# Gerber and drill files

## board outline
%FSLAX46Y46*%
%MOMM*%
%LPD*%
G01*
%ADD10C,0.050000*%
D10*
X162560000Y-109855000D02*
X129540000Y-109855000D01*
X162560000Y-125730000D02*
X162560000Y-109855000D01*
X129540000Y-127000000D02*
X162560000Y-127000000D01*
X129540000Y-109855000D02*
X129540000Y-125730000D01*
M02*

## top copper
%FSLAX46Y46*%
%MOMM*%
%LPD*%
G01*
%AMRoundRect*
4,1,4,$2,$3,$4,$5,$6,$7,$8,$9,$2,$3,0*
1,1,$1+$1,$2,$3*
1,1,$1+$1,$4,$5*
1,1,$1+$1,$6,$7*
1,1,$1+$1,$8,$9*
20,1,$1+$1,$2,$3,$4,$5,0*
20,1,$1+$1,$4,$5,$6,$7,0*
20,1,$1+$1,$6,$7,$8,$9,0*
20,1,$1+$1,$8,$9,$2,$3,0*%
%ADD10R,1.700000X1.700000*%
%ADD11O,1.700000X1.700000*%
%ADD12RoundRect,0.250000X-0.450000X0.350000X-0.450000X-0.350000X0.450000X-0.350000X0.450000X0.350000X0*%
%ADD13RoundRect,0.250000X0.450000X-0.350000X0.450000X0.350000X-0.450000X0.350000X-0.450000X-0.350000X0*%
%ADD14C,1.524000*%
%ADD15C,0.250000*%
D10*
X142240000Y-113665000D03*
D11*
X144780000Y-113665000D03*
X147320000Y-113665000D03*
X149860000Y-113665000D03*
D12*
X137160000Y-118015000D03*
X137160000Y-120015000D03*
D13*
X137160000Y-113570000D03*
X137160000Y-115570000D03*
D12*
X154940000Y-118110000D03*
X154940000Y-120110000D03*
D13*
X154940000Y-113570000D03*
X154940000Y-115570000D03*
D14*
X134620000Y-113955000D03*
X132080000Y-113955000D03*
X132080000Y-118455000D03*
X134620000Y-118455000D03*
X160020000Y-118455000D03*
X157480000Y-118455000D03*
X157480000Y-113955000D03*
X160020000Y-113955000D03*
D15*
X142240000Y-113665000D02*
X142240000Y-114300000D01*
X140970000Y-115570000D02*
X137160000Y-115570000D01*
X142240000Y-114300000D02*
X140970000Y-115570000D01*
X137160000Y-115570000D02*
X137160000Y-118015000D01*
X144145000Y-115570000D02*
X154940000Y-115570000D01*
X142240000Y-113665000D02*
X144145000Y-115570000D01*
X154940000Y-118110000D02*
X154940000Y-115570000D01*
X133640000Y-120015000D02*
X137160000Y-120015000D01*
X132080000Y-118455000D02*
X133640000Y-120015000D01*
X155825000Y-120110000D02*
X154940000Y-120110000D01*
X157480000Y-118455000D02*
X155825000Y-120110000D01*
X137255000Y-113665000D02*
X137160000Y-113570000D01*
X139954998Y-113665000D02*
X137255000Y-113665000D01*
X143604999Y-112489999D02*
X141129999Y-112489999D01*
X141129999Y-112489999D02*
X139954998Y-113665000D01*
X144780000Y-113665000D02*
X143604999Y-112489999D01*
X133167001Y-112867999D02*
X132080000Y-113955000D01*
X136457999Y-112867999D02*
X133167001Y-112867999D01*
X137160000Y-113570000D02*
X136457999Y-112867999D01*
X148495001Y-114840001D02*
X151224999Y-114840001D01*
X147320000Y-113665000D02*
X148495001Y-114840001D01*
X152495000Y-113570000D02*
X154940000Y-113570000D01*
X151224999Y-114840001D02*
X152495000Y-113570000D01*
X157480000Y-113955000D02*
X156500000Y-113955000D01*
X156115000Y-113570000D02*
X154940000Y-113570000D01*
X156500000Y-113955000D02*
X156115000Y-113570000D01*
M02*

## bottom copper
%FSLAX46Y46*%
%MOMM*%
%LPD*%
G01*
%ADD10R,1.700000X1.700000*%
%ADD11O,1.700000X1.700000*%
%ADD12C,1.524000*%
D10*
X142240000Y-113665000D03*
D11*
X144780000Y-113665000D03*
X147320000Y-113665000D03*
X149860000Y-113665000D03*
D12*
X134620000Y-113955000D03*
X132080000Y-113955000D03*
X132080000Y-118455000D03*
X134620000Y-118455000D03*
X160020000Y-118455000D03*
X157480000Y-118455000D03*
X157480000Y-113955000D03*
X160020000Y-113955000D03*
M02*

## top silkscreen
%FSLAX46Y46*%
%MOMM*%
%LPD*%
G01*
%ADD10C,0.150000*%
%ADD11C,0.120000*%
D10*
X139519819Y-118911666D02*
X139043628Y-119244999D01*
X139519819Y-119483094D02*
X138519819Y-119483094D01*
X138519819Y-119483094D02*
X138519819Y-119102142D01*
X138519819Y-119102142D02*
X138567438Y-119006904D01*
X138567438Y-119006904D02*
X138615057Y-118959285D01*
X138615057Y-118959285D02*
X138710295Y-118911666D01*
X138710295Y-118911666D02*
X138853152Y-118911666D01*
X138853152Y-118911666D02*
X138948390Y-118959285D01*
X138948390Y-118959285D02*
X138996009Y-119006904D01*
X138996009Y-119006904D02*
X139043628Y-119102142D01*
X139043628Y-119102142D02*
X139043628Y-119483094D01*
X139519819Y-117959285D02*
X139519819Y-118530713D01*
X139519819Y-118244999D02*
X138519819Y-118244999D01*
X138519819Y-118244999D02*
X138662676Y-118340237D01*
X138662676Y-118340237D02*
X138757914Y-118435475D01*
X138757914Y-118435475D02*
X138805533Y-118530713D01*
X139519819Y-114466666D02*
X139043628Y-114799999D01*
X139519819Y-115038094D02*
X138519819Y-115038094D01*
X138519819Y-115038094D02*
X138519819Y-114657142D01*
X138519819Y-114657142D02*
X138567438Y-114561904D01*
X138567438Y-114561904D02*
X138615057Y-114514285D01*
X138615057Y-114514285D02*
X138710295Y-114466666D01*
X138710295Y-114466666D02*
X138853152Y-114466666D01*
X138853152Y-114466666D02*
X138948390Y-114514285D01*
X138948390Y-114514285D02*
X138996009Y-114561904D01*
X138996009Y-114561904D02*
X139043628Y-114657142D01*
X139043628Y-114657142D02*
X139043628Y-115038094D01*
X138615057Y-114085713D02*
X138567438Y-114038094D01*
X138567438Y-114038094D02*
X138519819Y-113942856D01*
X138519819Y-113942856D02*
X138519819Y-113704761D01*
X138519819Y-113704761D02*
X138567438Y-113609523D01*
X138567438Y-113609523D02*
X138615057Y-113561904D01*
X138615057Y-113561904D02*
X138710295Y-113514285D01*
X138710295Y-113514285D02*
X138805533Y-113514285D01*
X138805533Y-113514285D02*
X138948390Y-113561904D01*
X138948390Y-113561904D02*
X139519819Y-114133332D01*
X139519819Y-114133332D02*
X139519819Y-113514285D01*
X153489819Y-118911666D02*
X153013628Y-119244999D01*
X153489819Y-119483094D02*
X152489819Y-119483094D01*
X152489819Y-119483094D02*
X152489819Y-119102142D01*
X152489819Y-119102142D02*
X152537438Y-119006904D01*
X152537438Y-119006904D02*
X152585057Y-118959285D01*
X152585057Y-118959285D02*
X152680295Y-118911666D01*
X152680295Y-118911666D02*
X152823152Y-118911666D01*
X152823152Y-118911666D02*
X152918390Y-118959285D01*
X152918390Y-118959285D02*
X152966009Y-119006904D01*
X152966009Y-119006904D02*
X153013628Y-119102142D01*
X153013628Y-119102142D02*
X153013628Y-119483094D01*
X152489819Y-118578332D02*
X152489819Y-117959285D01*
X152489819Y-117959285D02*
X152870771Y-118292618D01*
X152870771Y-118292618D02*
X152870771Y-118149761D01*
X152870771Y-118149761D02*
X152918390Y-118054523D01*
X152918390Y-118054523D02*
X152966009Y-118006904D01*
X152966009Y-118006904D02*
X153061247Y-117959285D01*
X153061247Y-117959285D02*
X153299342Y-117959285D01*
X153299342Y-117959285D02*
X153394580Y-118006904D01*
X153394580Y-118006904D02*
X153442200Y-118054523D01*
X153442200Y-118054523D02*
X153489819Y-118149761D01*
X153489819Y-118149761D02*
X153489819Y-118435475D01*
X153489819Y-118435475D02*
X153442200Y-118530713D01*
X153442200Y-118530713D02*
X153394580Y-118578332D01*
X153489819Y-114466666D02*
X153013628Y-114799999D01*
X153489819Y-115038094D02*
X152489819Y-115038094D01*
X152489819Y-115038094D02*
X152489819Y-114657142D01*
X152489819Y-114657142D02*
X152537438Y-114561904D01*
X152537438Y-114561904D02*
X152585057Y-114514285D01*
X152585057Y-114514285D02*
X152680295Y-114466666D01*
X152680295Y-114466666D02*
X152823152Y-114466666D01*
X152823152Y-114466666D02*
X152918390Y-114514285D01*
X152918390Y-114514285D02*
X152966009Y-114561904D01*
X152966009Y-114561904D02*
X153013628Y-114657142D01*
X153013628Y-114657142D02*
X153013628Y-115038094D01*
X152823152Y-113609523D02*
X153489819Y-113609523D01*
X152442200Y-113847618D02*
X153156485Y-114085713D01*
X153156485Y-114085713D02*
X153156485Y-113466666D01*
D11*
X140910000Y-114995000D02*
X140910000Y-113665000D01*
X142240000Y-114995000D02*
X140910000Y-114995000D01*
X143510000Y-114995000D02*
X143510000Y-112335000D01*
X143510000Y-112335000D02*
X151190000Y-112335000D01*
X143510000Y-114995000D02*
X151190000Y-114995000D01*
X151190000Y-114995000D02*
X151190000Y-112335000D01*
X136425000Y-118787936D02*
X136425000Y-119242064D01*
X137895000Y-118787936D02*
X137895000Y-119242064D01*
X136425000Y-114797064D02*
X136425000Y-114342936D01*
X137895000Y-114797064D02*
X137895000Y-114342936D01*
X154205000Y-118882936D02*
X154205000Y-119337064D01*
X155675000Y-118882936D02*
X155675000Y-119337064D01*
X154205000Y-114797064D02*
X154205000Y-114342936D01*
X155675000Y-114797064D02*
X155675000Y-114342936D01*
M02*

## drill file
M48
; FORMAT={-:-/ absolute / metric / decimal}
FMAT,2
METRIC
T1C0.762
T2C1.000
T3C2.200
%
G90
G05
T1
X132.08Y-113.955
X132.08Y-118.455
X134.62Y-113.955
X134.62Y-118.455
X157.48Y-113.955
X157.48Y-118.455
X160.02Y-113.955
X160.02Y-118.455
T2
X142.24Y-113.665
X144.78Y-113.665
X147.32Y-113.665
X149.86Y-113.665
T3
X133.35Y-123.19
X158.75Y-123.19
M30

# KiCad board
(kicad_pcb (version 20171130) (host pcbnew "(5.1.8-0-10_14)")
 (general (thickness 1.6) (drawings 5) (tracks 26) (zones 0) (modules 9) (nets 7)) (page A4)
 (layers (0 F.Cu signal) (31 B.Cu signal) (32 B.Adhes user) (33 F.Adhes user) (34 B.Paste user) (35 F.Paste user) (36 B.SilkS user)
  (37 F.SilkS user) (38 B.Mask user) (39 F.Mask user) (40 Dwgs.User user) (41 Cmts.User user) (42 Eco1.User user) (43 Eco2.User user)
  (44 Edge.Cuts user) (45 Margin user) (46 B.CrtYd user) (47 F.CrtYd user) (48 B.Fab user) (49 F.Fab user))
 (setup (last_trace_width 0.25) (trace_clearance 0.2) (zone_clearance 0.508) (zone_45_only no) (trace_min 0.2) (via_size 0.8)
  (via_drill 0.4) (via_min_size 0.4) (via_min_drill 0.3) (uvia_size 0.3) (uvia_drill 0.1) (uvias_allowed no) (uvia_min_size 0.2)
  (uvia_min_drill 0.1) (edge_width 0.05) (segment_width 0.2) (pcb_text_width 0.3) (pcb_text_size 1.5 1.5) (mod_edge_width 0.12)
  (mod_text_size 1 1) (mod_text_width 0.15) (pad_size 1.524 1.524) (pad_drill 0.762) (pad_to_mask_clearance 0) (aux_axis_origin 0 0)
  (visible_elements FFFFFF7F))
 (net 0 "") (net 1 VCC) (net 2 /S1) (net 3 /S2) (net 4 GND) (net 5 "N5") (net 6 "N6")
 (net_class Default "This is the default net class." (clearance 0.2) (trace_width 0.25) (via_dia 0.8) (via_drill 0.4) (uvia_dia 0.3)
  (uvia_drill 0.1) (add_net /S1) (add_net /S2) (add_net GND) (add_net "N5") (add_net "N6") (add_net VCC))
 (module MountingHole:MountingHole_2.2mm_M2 (layer F.Cu) (at 133.35 123.19)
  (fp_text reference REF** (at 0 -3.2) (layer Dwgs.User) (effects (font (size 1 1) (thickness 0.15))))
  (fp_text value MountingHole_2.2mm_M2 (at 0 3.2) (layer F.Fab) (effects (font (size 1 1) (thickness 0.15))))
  (pad 1 np_thru_hole circle (at 0 0) (size 2.2 2.2) (drill 2.2) (layers *.Cu *.Mask)))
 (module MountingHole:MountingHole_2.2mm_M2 (layer F.Cu) (at 158.75 123.19)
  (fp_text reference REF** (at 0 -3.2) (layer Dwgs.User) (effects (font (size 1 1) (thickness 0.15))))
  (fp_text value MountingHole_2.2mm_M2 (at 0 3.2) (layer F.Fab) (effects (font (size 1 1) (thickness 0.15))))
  (pad 1 np_thru_hole circle (at 0 0) (size 2.2 2.2) (drill 2.2) (layers *.Cu *.Mask)))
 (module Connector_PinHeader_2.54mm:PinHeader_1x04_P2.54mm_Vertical (layer F.Cu) (at 142.24 113.665 90)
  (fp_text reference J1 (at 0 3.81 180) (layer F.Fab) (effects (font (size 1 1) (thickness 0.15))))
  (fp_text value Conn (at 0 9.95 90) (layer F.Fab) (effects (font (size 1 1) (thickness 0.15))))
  (fp_line (start -1.33 -1.33) (end 0 -1.33) (layer F.SilkS) (width 0.12))
  (fp_line (start -1.33 0) (end -1.33 -1.33) (layer F.SilkS) (width 0.12))
  (fp_line (start -1.33 1.27) (end 1.33 1.27) (layer F.SilkS) (width 0.12))
  (fp_line (start 1.33 1.27) (end 1.33 8.95) (layer F.SilkS) (width 0.12))
  (fp_line (start -1.33 1.27) (end -1.33 8.95) (layer F.SilkS) (width 0.12))
  (fp_line (start -1.33 8.95) (end 1.33 8.95) (layer F.SilkS) (width 0.12))
  (pad 1 thru_hole rect (at 0 0 90) (size 1.7 1.7) (drill 1) (layers *.Cu *.Mask) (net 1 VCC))
  (pad 2 thru_hole oval (at 0 2.54 90) (size 1.7 1.7) (drill 1) (layers *.Cu *.Mask) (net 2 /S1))
  (pad 3 thru_hole oval (at 0 5.08 90) (size 1.7 1.7) (drill 1) (layers *.Cu *.Mask) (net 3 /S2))
  (pad 4 thru_hole oval (at 0 7.62 90) (size 1.7 1.7) (drill 1) (layers *.Cu *.Mask) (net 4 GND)))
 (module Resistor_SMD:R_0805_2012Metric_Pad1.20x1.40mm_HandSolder (layer F.Cu) (at 137.16 119.015 270)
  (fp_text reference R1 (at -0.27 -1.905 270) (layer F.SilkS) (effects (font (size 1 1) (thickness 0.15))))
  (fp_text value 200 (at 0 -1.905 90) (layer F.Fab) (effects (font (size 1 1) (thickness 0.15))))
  (fp_line (start -0.227064 0.735) (end 0.227064 0.735) (layer F.SilkS) (width 0.12))
  (fp_line (start -0.227064 -0.735) (end 0.227064 -0.735) (layer F.SilkS) (width 0.12))
  (pad 1 smd roundrect (at -1 0 270) (size 1.2 1.4) (layers F.Cu F.Paste F.Mask) (roundrect_rratio 0.208333) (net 1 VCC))
  (pad 2 smd roundrect (at 1 0 270) (size 1.2 1.4) (layers F.Cu F.Paste F.Mask) (roundrect_rratio 0.208333) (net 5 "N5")))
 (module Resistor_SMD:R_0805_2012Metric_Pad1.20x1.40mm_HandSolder (layer F.Cu) (at 137.16 114.57 90)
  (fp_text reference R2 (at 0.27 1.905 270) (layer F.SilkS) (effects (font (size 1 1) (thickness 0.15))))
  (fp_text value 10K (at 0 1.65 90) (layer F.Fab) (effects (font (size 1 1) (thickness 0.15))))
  (fp_line (start -0.227064 -0.735) (end 0.227064 -0.735) (layer F.SilkS) (width 0.12))
  (fp_line (start -0.227064 0.735) (end 0.227064 0.735) (layer F.SilkS) (width 0.12))
  (pad 2 smd roundrect (at 1 0 90) (size 1.2 1.4) (layers F.Cu F.Paste F.Mask) (roundrect_rratio 0.208333) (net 2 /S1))
  (pad 1 smd roundrect (at -1 0 90) (size 1.2 1.4) (layers F.Cu F.Paste F.Mask) (roundrect_rratio 0.208333) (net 1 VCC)))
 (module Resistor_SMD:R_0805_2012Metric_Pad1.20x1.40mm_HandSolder (layer F.Cu) (at 154.94 119.11 270)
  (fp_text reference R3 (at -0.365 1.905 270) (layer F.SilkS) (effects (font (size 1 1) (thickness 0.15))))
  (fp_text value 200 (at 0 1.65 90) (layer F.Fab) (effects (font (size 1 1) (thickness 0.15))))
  (fp_line (start -0.227064 0.735) (end 0.227064 0.735) (layer F.SilkS) (width 0.12))
  (fp_line (start -0.227064 -0.735) (end 0.227064 -0.735) (layer F.SilkS) (width 0.12))
  (pad 1 smd roundrect (at -1 0 270) (size 1.2 1.4) (layers F.Cu F.Paste F.Mask) (roundrect_rratio 0.208333) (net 1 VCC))
  (pad 2 smd roundrect (at 1 0 270) (size 1.2 1.4) (layers F.Cu F.Paste F.Mask) (roundrect_rratio 0.208333) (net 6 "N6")))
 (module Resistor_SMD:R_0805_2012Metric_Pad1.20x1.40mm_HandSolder (layer F.Cu) (at 154.94 114.57 90)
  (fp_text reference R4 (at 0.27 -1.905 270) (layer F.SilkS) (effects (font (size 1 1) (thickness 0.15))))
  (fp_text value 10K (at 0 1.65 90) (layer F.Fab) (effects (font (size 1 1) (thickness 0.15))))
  (fp_line (start -0.227064 -0.735) (end 0.227064 -0.735) (layer F.SilkS) (width 0.12))
  (fp_line (start -0.227064 0.735) (end 0.227064 0.735) (layer F.SilkS) (width 0.12))
  (pad 2 smd roundrect (at 1 0 90) (size 1.2 1.4) (layers F.Cu F.Paste F.Mask) (roundrect_rratio 0.208333) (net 3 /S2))
  (pad 1 smd roundrect (at -1 0 90) (size 1.2 1.4) (layers F.Cu F.Paste F.Mask) (roundrect_rratio 0.208333) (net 1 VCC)))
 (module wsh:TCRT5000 (layer B.Cu) (at 133.35 116.205 270)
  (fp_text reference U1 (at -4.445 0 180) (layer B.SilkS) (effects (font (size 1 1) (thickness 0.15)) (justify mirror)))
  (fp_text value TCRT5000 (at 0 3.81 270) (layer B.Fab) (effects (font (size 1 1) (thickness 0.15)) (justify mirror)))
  (pad 4 thru_hole circle (at -2.25 -1.27 270) (size 1.524 1.524) (drill 0.762) (layers *.Cu *.Mask) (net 4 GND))
  (pad 3 thru_hole circle (at -2.25 1.27 270) (size 1.524 1.524) (drill 0.762) (layers *.Cu *.Mask) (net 2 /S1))
  (pad 2 thru_hole circle (at 2.25 1.27 270) (size 1.524 1.524) (drill 0.762) (layers *.Cu *.Mask) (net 5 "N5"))
  (pad 1 thru_hole circle (at 2.25 -1.27 270) (size 1.524 1.524) (drill 0.762) (layers *.Cu *.Mask) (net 4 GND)))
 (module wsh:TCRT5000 (layer B.Cu) (at 158.75 116.205 270)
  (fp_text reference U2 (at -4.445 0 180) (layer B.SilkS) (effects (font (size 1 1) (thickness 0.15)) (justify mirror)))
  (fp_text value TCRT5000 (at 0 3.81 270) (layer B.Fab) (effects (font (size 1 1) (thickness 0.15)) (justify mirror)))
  (pad 1 thru_hole circle (at 2.25 -1.27 270) (size 1.524 1.524) (drill 0.762) (layers *.Cu *.Mask) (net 4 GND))
  (pad 2 thru_hole circle (at 2.25 1.27 270) (size 1.524 1.524) (drill 0.762) (layers *.Cu *.Mask) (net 6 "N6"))
  (pad 3 thru_hole circle (at -2.25 1.27 270) (size 1.524 1.524) (drill 0.762) (layers *.Cu *.Mask) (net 3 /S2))
  (pad 4 thru_hole circle (at -2.25 -1.27 270) (size 1.524 1.524) (drill 0.762) (layers *.Cu *.Mask) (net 4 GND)))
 (gr_line (start 162.56 109.855) (end 129.54 109.855) (layer Edge.Cuts) (width 0.05))
 (gr_line (start 162.56 125.73) (end 162.56 109.855) (layer Edge.Cuts) (width 0.05))
 (gr_line (start 129.54 127) (end 162.56 127) (layer Edge.Cuts) (width 0.05))
 (gr_line (start 129.54 109.855) (end 129.54 125.73) (layer Edge.Cuts) (width 0.05))
 (segment (start 142.24 113.665) (end 142.24 114.3) (width 0.25) (layer F.Cu) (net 1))
 (segment (start 140.97 115.57) (end 137.16 115.57) (width 0.25) (layer F.Cu) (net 1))
 (segment (start 142.24 114.3) (end 140.97 115.57) (width 0.25) (layer F.Cu) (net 1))
 (segment (start 137.16 115.57) (end 137.16 118.015) (width 0.25) (layer F.Cu) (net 1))
 (segment (start 144.145 115.57) (end 154.94 115.57) (width 0.25) (layer F.Cu) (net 1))
 (segment (start 142.24 113.665) (end 144.145 115.57) (width 0.25) (layer F.Cu) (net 1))
 (segment (start 154.94 118.11) (end 154.94 115.57) (width 0.25) (layer F.Cu) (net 1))
 (segment (start 133.64 120.015) (end 137.16 120.015) (width 0.25) (layer F.Cu) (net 5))
 (segment (start 132.08 118.455) (end 133.64 120.015) (width 0.25) (layer F.Cu) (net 5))
 (segment (start 155.825 120.11) (end 154.94 120.11) (width 0.25) (layer F.Cu) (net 6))
 (segment (start 157.48 118.455) (end 155.825 120.11) (width 0.25) (layer F.Cu) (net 6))
 (segment (start 137.255 113.665) (end 137.16 113.57) (width 0.25) (layer F.Cu) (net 2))
 (segment (start 139.954998 113.665) (end 137.255 113.665) (width 0.25) (layer F.Cu) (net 2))
 (segment (start 143.604999 112.489999) (end 141.129999 112.489999) (width 0.25) (layer F.Cu) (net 2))
 (segment (start 141.129999 112.489999) (end 139.954998 113.665) (width 0.25) (layer F.Cu) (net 2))
 (segment (start 144.78 113.665) (end 143.604999 112.489999) (width 0.25) (layer F.Cu) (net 2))
 (segment (start 133.167001 112.867999) (end 132.08 113.955) (width 0.25) (layer F.Cu) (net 2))
 (segment (start 136.457999 112.867999) (end 133.167001 112.867999) (width 0.25) (layer F.Cu) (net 2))
 (segment (start 137.16 113.57) (end 136.457999 112.867999) (width 0.25) (layer F.Cu) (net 2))
 (segment (start 148.495001 114.840001) (end 151.224999 114.840001) (width 0.25) (layer F.Cu) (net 3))
 (segment (start 147.32 113.665) (end 148.495001 114.840001) (width 0.25) (layer F.Cu) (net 3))
 (segment (start 152.495 113.57) (end 154.94 113.57) (width 0.25) (layer F.Cu) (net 3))
 (segment (start 151.224999 114.840001) (end 152.495 113.57) (width 0.25) (layer F.Cu) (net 3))
 (segment (start 157.48 113.955) (end 156.5 113.955) (width 0.25) (layer F.Cu) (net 3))
 (segment (start 156.115 113.57) (end 154.94 113.57) (width 0.25) (layer F.Cu) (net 3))
 (segment (start 156.5 113.955) (end 156.115 113.57) (width 0.25) (layer F.Cu) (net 3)))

